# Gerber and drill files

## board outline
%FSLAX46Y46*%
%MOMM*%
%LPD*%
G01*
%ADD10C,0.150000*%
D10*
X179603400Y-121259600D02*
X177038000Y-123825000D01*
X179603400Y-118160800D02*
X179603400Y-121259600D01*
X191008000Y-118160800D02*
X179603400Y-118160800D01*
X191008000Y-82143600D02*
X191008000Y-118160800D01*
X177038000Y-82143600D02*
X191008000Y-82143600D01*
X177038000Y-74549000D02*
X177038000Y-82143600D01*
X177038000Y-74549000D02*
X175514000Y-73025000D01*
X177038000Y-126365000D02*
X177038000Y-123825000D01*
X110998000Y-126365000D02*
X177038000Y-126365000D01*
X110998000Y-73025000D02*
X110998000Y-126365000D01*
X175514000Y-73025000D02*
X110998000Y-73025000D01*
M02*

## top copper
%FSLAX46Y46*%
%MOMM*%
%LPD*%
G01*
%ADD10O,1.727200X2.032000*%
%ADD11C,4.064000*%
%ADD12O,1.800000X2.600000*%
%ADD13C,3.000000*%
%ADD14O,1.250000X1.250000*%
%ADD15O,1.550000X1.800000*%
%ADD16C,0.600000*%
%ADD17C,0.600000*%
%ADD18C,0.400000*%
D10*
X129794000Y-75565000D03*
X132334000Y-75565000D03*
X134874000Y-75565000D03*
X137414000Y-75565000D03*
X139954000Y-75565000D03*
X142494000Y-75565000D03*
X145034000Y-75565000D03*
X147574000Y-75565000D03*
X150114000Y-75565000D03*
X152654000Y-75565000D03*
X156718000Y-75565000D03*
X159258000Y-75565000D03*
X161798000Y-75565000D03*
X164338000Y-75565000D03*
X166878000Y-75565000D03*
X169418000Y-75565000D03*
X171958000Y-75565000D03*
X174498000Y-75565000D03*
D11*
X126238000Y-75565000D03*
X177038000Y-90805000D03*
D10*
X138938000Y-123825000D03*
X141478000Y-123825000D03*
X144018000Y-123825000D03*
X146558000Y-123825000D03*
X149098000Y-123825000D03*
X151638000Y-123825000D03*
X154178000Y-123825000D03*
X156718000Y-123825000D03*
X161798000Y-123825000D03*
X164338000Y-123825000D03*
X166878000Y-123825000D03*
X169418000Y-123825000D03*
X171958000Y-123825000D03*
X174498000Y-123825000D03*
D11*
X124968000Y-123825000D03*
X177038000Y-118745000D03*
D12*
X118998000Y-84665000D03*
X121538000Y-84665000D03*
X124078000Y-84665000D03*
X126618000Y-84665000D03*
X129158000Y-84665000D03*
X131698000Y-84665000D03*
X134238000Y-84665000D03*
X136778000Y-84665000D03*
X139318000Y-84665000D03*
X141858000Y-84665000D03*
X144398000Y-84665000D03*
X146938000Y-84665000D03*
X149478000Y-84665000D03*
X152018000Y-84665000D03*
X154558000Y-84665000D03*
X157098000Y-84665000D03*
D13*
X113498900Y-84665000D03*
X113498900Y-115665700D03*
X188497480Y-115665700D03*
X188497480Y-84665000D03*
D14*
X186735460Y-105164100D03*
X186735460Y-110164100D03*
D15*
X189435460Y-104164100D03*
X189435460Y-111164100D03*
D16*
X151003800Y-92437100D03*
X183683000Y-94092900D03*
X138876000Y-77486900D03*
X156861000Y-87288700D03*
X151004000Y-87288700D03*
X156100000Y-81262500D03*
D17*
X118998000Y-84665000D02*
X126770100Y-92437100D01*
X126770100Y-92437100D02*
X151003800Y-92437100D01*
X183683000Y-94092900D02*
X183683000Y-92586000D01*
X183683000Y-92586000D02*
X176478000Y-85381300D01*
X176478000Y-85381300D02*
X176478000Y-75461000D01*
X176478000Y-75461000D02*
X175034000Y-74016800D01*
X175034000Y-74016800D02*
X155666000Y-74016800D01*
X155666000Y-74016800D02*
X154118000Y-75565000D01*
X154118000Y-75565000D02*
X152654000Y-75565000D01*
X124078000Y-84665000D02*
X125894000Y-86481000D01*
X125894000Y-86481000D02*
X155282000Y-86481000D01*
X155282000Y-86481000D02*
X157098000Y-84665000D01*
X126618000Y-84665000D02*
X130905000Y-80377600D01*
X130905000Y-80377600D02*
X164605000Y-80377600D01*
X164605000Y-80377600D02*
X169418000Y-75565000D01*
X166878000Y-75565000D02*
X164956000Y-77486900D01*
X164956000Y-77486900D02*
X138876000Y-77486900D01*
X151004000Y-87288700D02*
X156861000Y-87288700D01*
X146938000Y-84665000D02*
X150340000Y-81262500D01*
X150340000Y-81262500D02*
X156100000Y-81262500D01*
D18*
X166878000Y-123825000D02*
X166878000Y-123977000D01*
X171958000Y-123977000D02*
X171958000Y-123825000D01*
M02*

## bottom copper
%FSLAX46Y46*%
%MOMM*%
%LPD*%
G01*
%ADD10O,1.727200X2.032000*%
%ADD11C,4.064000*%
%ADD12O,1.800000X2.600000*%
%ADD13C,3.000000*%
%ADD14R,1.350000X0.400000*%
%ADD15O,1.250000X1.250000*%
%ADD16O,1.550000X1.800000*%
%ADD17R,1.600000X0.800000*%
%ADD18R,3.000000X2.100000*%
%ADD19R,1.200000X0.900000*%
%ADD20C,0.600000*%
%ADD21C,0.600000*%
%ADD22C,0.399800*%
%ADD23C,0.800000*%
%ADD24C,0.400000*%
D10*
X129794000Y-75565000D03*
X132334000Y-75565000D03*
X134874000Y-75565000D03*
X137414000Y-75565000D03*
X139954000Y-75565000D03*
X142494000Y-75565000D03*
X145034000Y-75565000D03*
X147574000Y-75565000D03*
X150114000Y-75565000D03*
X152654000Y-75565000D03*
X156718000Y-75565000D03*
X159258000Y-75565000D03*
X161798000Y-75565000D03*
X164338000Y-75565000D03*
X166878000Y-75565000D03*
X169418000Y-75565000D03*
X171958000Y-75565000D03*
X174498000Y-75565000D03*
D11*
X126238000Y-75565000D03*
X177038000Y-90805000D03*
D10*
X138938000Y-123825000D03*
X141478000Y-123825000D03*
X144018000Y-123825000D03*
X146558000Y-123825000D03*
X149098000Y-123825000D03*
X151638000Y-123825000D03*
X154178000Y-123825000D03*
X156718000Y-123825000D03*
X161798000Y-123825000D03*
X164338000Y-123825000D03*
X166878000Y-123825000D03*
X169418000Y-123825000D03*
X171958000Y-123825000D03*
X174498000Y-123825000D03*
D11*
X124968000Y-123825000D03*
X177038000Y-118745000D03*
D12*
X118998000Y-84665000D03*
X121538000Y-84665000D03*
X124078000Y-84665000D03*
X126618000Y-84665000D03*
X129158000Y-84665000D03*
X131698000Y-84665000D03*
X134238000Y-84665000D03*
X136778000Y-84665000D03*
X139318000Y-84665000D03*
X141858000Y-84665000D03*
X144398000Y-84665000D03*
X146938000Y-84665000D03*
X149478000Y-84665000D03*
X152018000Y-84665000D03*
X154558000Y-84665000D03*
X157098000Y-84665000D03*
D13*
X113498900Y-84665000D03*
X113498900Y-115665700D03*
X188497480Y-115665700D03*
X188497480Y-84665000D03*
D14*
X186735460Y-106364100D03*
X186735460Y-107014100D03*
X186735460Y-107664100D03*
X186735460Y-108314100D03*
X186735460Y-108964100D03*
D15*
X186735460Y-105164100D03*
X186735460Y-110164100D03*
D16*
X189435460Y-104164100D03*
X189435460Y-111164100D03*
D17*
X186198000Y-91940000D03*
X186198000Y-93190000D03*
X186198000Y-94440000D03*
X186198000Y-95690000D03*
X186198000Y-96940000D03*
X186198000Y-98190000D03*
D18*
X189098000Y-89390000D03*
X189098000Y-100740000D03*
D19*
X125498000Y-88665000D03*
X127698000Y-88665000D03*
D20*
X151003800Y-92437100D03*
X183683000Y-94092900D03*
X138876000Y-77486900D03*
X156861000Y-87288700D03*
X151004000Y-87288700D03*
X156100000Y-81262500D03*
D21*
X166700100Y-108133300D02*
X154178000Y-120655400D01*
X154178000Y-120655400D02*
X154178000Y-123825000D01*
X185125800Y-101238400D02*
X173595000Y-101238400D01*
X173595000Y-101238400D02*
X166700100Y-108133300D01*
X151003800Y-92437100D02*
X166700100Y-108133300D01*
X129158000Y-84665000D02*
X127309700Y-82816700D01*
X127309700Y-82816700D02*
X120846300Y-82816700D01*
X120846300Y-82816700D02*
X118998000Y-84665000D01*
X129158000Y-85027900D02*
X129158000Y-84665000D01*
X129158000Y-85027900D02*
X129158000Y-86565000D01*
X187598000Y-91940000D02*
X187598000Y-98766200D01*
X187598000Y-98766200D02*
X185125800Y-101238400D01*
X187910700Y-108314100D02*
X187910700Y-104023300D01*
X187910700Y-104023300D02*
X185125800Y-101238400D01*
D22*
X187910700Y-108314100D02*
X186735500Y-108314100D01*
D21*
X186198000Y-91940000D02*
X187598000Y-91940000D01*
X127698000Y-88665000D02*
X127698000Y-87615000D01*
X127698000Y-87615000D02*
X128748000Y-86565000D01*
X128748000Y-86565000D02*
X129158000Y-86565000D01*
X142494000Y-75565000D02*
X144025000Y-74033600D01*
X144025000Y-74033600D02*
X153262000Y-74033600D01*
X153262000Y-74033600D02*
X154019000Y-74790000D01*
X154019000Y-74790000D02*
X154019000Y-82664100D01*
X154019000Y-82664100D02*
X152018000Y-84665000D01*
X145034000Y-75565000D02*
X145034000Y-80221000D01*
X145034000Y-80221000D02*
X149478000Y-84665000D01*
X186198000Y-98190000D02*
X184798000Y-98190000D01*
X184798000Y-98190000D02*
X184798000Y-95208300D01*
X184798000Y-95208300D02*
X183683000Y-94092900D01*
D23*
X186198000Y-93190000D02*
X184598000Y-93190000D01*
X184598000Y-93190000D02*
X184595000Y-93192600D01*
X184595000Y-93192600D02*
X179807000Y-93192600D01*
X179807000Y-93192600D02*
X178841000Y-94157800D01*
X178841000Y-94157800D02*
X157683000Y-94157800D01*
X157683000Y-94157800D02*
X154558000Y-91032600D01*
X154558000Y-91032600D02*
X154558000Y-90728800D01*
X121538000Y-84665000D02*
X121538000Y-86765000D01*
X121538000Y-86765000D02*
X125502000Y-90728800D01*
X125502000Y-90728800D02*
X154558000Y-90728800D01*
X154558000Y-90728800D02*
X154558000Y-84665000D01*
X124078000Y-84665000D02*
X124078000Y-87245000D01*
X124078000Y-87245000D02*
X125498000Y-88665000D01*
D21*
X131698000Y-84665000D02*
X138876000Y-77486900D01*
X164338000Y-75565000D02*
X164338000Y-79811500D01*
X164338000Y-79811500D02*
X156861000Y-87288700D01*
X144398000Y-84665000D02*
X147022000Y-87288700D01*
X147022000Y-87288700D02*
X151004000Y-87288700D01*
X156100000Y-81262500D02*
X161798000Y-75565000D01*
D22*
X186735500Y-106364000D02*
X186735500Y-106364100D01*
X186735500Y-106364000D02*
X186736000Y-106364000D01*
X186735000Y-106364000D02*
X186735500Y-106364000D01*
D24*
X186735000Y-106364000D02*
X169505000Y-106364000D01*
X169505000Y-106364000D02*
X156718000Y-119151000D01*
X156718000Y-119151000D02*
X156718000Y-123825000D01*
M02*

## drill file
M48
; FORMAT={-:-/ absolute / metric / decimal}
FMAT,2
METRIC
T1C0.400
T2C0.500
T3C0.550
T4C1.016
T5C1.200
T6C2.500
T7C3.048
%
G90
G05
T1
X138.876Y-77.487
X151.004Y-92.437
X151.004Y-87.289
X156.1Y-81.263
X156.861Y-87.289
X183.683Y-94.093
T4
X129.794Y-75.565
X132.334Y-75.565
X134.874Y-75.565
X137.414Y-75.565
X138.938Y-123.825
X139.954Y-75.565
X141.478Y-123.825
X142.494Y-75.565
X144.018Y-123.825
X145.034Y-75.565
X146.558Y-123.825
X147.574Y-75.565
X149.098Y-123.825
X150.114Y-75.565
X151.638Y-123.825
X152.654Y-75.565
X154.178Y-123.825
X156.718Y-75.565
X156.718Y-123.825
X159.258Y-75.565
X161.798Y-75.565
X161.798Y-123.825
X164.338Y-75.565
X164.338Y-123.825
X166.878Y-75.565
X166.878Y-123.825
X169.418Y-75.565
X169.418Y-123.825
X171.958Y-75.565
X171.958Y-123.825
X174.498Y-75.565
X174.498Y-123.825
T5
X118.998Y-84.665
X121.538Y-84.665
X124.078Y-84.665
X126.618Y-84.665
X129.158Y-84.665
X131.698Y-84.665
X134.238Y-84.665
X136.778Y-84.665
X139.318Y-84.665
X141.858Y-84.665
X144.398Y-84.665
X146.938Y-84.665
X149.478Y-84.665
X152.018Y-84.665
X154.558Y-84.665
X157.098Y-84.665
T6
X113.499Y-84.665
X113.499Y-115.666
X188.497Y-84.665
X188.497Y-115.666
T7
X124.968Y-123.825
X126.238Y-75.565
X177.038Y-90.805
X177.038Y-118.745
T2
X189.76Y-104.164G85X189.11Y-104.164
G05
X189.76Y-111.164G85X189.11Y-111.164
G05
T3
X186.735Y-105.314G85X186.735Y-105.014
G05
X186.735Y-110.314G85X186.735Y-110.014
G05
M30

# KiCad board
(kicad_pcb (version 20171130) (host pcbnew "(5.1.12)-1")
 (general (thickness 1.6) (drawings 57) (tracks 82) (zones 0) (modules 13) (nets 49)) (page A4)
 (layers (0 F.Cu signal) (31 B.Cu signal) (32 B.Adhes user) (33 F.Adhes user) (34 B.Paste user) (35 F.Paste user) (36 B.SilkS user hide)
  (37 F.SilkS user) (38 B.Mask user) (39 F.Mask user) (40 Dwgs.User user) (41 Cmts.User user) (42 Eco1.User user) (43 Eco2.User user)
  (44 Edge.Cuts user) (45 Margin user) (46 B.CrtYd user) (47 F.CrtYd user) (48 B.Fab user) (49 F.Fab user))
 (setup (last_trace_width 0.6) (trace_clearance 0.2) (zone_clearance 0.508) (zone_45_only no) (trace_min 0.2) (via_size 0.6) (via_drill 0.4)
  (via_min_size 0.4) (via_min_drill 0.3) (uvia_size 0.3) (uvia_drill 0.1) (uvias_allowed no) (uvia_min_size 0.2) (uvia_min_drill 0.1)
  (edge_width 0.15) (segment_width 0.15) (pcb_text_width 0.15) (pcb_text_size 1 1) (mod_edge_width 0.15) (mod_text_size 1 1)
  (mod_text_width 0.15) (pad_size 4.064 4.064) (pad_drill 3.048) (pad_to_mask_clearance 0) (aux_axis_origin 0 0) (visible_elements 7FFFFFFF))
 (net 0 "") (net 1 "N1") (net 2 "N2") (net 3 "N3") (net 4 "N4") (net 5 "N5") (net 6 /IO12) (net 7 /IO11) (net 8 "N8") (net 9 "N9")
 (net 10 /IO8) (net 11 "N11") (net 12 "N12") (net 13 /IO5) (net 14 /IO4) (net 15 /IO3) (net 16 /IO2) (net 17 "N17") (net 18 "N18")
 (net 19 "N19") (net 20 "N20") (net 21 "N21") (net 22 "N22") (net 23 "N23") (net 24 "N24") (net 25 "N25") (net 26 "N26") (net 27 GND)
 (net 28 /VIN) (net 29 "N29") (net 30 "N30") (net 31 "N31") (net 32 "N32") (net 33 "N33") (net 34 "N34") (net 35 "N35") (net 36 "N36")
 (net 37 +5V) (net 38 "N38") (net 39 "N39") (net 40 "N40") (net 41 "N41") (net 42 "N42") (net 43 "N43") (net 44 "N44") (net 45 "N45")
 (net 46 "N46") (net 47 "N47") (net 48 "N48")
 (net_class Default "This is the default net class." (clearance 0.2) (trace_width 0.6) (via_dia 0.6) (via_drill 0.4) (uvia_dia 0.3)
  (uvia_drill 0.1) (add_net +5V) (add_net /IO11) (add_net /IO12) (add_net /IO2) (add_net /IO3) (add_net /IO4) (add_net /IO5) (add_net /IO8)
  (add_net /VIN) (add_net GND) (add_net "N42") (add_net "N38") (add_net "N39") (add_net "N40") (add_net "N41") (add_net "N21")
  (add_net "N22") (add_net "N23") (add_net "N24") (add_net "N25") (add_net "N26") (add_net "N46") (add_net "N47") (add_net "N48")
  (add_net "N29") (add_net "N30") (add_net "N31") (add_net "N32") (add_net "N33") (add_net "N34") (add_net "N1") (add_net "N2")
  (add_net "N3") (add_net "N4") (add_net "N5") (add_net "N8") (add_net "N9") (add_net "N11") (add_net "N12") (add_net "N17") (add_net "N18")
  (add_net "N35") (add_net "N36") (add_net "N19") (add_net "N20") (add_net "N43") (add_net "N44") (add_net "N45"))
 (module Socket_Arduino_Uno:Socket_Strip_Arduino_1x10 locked (layer F.Cu) (at 129.794 75.565)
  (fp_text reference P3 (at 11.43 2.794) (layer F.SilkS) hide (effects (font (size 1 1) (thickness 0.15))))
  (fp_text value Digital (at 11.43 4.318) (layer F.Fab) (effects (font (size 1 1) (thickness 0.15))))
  (pad 1 thru_hole oval (at 0 0) (size 1.7272 2.032) (drill 1.016) (layers *.Cu *.Mask F.SilkS) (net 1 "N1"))
  (pad 2 thru_hole oval (at 2.54 0) (size 1.7272 2.032) (drill 1.016) (layers *.Cu *.Mask F.SilkS) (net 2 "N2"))
  (pad 3 thru_hole oval (at 5.08 0) (size 1.7272 2.032) (drill 1.016) (layers *.Cu *.Mask F.SilkS) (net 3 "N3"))
  (pad 4 thru_hole oval (at 7.62 0) (size 1.7272 2.032) (drill 1.016) (layers *.Cu *.Mask F.SilkS) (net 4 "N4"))
  (pad 5 thru_hole oval (at 10.16 0) (size 1.7272 2.032) (drill 1.016) (layers *.Cu *.Mask F.SilkS) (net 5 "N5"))
  (pad 6 thru_hole oval (at 12.7 0) (size 1.7272 2.032) (drill 1.016) (layers *.Cu *.Mask F.SilkS) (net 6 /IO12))
  (pad 7 thru_hole oval (at 15.24 0) (size 1.7272 2.032) (drill 1.016) (layers *.Cu *.Mask F.SilkS) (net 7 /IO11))
  (pad 8 thru_hole oval (at 17.78 0) (size 1.7272 2.032) (drill 1.016) (layers *.Cu *.Mask F.SilkS) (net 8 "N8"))
  (pad 9 thru_hole oval (at 20.32 0) (size 1.7272 2.032) (drill 1.016) (layers *.Cu *.Mask F.SilkS) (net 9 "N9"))
  (pad 10 thru_hole oval (at 22.86 0) (size 1.7272 2.032) (drill 1.016) (layers *.Cu *.Mask F.SilkS) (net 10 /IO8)))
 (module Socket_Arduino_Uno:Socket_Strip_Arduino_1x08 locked (layer F.Cu) (at 156.718 75.565)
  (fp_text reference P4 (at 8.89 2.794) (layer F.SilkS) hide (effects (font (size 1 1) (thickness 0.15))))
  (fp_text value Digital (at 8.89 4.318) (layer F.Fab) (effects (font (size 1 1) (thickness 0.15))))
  (pad 1 thru_hole oval (at 0 0) (size 1.7272 2.032) (drill 1.016) (layers *.Cu *.Mask F.SilkS) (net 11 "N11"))
  (pad 2 thru_hole oval (at 2.54 0) (size 1.7272 2.032) (drill 1.016) (layers *.Cu *.Mask F.SilkS) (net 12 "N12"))
  (pad 3 thru_hole oval (at 5.08 0) (size 1.7272 2.032) (drill 1.016) (layers *.Cu *.Mask F.SilkS) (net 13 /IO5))
  (pad 4 thru_hole oval (at 7.62 0) (size 1.7272 2.032) (drill 1.016) (layers *.Cu *.Mask F.SilkS) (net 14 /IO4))
  (pad 5 thru_hole oval (at 10.16 0) (size 1.7272 2.032) (drill 1.016) (layers *.Cu *.Mask F.SilkS) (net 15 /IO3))
  (pad 6 thru_hole oval (at 12.7 0) (size 1.7272 2.032) (drill 1.016) (layers *.Cu *.Mask F.SilkS) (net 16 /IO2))
  (pad 7 thru_hole oval (at 15.24 0) (size 1.7272 2.032) (drill 1.016) (layers *.Cu *.Mask F.SilkS) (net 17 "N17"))
  (pad 8 thru_hole oval (at 17.78 0) (size 1.7272 2.032) (drill 1.016) (layers *.Cu *.Mask F.SilkS) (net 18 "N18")))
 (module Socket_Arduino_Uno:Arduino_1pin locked (layer F.Cu) (at 126.238 75.565)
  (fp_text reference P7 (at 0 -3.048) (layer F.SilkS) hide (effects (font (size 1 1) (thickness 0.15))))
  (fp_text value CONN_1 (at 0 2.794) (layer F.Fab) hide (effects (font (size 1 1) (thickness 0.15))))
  (pad 1 thru_hole circle (at 0 0) (size 4.064 4.064) (drill 3.048) (layers *.Cu *.Mask F.SilkS) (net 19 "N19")))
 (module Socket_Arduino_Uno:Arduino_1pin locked (layer F.Cu) (at 177.038 90.805)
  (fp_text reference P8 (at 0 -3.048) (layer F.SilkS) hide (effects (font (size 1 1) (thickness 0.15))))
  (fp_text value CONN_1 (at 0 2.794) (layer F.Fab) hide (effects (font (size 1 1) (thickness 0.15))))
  (pad 1 thru_hole circle (at 0 0) (size 4.064 4.064) (drill 3.048) (layers *.Cu *.Mask F.SilkS) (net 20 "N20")))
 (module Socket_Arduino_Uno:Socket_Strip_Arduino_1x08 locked (layer F.Cu) (at 138.938 123.825)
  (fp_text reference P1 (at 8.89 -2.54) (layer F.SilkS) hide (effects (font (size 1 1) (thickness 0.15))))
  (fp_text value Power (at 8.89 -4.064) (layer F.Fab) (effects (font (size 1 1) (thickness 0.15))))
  (pad 1 thru_hole oval (at 0 0) (size 1.7272 2.032) (drill 1.016) (layers *.Cu *.Mask F.SilkS) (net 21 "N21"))
  (pad 2 thru_hole oval (at 2.54 0) (size 1.7272 2.032) (drill 1.016) (layers *.Cu *.Mask F.SilkS) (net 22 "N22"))
  (pad 3 thru_hole oval (at 5.08 0) (size 1.7272 2.032) (drill 1.016) (layers *.Cu *.Mask F.SilkS) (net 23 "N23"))
  (pad 4 thru_hole oval (at 7.62 0) (size 1.7272 2.032) (drill 1.016) (layers *.Cu *.Mask F.SilkS) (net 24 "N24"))
  (pad 5 thru_hole oval (at 10.16 0) (size 1.7272 2.032) (drill 1.016) (layers *.Cu *.Mask F.SilkS) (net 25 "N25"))
  (pad 6 thru_hole oval (at 12.7 0) (size 1.7272 2.032) (drill 1.016) (layers *.Cu *.Mask F.SilkS) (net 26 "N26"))
  (pad 7 thru_hole oval (at 15.24 0) (size 1.7272 2.032) (drill 1.016) (layers *.Cu *.Mask F.SilkS) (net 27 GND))
  (pad 8 thru_hole oval (at 17.78 0) (size 1.7272 2.032) (drill 1.016) (layers *.Cu *.Mask F.SilkS) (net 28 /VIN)))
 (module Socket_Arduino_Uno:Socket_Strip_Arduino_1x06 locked (layer F.Cu) (at 161.798 123.825)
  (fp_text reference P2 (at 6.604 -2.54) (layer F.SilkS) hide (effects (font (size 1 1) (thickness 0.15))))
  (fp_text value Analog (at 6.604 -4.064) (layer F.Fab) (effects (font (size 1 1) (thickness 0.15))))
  (pad 1 thru_hole oval (at 0 0) (size 1.7272 2.032) (drill 1.016) (layers *.Cu *.Mask F.SilkS) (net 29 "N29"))
  (pad 2 thru_hole oval (at 2.54 0) (size 1.7272 2.032) (drill 1.016) (layers *.Cu *.Mask F.SilkS) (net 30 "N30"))
  (pad 3 thru_hole oval (at 5.08 0) (size 1.7272 2.032) (drill 1.016) (layers *.Cu *.Mask F.SilkS) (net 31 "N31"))
  (pad 4 thru_hole oval (at 7.62 0) (size 1.7272 2.032) (drill 1.016) (layers *.Cu *.Mask F.SilkS) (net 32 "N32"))
  (pad 5 thru_hole oval (at 10.16 0) (size 1.7272 2.032) (drill 1.016) (layers *.Cu *.Mask F.SilkS) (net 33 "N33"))
  (pad 6 thru_hole oval (at 12.7 0) (size 1.7272 2.032) (drill 1.016) (layers *.Cu *.Mask F.SilkS) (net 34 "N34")))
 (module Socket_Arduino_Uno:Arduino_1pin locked (layer F.Cu) (at 124.968 123.825)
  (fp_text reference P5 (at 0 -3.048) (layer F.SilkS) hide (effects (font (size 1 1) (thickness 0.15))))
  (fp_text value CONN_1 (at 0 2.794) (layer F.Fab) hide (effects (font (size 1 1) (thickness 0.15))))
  (pad 1 thru_hole circle (at 0 0) (size 4.064 4.064) (drill 3.048) (layers *.Cu *.Mask F.SilkS) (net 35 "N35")))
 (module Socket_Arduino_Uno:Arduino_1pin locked (layer F.Cu) (at 177.038 118.745)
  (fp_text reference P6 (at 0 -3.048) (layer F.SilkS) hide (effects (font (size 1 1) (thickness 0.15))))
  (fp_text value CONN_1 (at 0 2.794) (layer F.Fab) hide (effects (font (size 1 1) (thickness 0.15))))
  (pad 1 thru_hole circle (at 0 0) (size 4.064 4.064) (drill 3.048) (layers *.Cu *.Mask F.SilkS) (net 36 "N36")))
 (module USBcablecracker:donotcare (layer B.Cu) (at 164.1856 107.3658 180)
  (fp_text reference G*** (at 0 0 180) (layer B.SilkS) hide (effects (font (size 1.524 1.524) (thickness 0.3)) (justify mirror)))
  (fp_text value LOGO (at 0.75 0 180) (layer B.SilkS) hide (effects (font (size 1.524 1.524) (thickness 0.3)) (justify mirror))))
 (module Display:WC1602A (layer F.Cu) (at 118.998 84.665)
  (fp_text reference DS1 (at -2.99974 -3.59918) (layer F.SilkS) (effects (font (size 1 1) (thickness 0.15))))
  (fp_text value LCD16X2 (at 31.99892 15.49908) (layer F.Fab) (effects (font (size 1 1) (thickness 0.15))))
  (pad 1 thru_hole oval (at 0 0) (size 1.8 2.6) (drill 1.2) (layers *.Cu *.Mask F.SilkS) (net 27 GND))
  (pad 2 thru_hole oval (at 2.54 0) (size 1.8 2.6) (drill 1.2) (layers *.Cu *.Mask F.SilkS) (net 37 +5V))
  (pad 3 thru_hole oval (at 5.08 0) (size 1.8 2.6) (drill 1.2) (layers *.Cu *.Mask F.SilkS) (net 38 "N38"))
  (pad 4 thru_hole oval (at 7.62 0) (size 1.8 2.6) (drill 1.2) (layers *.Cu *.Mask F.SilkS) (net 16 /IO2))
  (pad 5 thru_hole oval (at 10.16 0) (size 1.8 2.6) (drill 1.2) (layers *.Cu *.Mask F.SilkS) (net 27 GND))
  (pad 6 thru_hole oval (at 12.7 0) (size 1.8 2.6) (drill 1.2) (layers *.Cu *.Mask F.SilkS) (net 15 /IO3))
  (pad 7 thru_hole oval (at 15.24 0) (size 1.8 2.6) (drill 1.2) (layers *.Cu *.Mask F.SilkS) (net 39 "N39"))
  (pad 8 thru_hole oval (at 17.78 0) (size 1.8 2.6) (drill 1.2) (layers *.Cu *.Mask F.SilkS) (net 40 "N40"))
  (pad 9 thru_hole oval (at 20.32 0) (size 1.8 2.6) (drill 1.2) (layers *.Cu *.Mask F.SilkS) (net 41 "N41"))
  (pad 10 thru_hole oval (at 22.86 0) (size 1.8 2.6) (drill 1.2) (layers *.Cu *.Mask F.SilkS) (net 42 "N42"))
  (pad 11 thru_hole oval (at 25.4 0) (size 1.8 2.6) (drill 1.2) (layers *.Cu *.Mask F.SilkS) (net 14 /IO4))
  (pad 12 thru_hole oval (at 27.94 0) (size 1.8 2.6) (drill 1.2) (layers *.Cu *.Mask F.SilkS) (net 13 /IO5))
  (pad 13 thru_hole oval (at 30.48 0) (size 1.8 2.6) (drill 1.2) (layers *.Cu *.Mask F.SilkS) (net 7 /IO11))
  (pad 14 thru_hole oval (at 33.02 0) (size 1.8 2.6) (drill 1.2) (layers *.Cu *.Mask F.SilkS) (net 6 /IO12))
  (pad 15 thru_hole oval (at 35.56 0) (size 1.8 2.6) (drill 1.2) (layers *.Cu *.Mask F.SilkS) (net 37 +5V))
  (pad 16 thru_hole oval (at 38.1 0) (size 1.8 2.6) (drill 1.2) (layers *.Cu *.Mask F.SilkS) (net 38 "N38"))
  (pad 0 thru_hole circle (at -5.4991 0) (size 3 3) (drill 2.5) (layers *.Cu *.Mask F.SilkS))
  (pad 0 thru_hole circle (at -5.4991 31.0007) (size 3 3) (drill 2.5) (layers *.Cu *.Mask F.SilkS))
  (pad 0 thru_hole circle (at 69.49948 31.0007) (size 3 3) (drill 2.5) (layers *.Cu *.Mask F.SilkS))
  (pad 0 thru_hole circle (at 69.49948 0) (size 3 3) (drill 2.5) (layers *.Cu *.Mask F.SilkS)))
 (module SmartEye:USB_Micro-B (layer B.Cu) (at 188.298 107.665 270)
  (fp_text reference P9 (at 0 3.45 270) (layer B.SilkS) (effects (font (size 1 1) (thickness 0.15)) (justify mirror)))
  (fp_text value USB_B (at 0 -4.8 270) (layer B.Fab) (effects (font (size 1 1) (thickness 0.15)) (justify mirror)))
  (pad 1 smd rect (at -1.3009 1.56254 180) (size 1.35 0.4) (layers B.Cu B.Paste B.Mask) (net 28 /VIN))
  (pad 2 smd rect (at -0.6509 1.56254 180) (size 1.35 0.4) (layers B.Cu B.Paste B.Mask) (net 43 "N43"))
  (pad 3 smd rect (at -0.0009 1.56254 180) (size 1.35 0.4) (layers B.Cu B.Paste B.Mask) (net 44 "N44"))
  (pad 4 smd rect (at 0.6491 1.56254 180) (size 1.35 0.4) (layers B.Cu B.Paste B.Mask) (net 27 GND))
  (pad 5 smd rect (at 1.2991 1.56254 180) (size 1.35 0.4) (layers B.Cu B.Paste B.Mask) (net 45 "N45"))
  (pad 6 thru_hole oval (at -2.5009 1.56254 180) (size 1.25 1.25) (drill oval 0.55 0.85) (layers *.Cu *.Mask B.SilkS))
  (pad 6 thru_hole oval (at 2.4991 1.56254 180) (size 1.25 1.25) (drill oval 0.55 0.85) (layers *.Cu *.Mask B.SilkS))
  (pad 6 thru_hole oval (at -3.5009 -1.13746 180) (size 1.55 1.8) (drill oval 1.15 0.5) (layers *.Cu *.Mask B.SilkS))
  (pad 6 thru_hole oval (at 3.4991 -1.13746 180) (size 1.55 1.8) (drill oval 1.15 0.5) (layers *.Cu *.Mask B.SilkS)))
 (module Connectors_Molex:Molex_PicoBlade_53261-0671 (layer B.Cu) (at 189.098 95.065 270)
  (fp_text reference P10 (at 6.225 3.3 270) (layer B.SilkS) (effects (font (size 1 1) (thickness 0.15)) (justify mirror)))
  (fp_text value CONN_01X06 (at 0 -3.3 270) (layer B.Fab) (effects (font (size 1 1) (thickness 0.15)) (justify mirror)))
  (pad 1 smd rect (at -3.125 2.9 270) (size 0.8 1.6) (layers B.Cu B.Paste B.Mask) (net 27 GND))
  (pad 2 smd rect (at -1.875 2.9 270) (size 0.8 1.6) (layers B.Cu B.Paste B.Mask) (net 37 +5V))
  (pad 3 smd rect (at -0.625 2.9 270) (size 0.8 1.6) (layers B.Cu B.Paste B.Mask) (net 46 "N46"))
  (pad 4 smd rect (at 0.625 2.9 270) (size 0.8 1.6) (layers B.Cu B.Paste B.Mask) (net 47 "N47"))
  (pad 5 smd rect (at 1.875 2.9 270) (size 0.8 1.6) (layers B.Cu B.Paste B.Mask) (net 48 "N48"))
  (pad 6 smd rect (at 3.125 2.9 270) (size 0.8 1.6) (layers B.Cu B.Paste B.Mask) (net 10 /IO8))
  (pad "" smd rect (at -5.675 0 270) (size 2.1 3) (layers B.Cu B.Paste B.Mask))
  (pad "" smd rect (at 5.675 0 270) (size 2.1 3) (layers B.Cu B.Paste B.Mask)))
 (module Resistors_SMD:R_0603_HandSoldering (layer B.Cu) (at 126.598 88.665)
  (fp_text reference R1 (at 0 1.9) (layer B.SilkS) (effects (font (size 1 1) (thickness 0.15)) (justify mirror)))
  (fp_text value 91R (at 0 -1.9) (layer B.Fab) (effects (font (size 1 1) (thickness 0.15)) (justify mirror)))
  (pad 1 smd rect (at -1.1 0) (size 1.2 0.9) (layers B.Cu B.Paste B.Mask) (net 38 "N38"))
  (pad 2 smd rect (at 1.1 0) (size 1.2 0.9) (layers B.Cu B.Paste B.Mask) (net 27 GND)))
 (gr_line (start 179.6034 121.2596) (end 177.038 123.825) (angle 90) (layer Edge.Cuts) (width 0.15))
 (gr_line (start 179.6034 118.1608) (end 179.6034 121.2596) (angle 90) (layer Edge.Cuts) (width 0.15))
 (gr_line (start 191.008 118.1608) (end 179.6034 118.1608) (angle 90) (layer Edge.Cuts) (width 0.15))
 (gr_line (start 191.008 82.1436) (end 191.008 118.1608) (angle 90) (layer Edge.Cuts) (width 0.15))
 (gr_line (start 177.038 82.1436) (end 191.008 82.1436) (angle 90) (layer Edge.Cuts) (width 0.15))
 (gr_line (start 177.038 74.549) (end 177.038 82.1436) (angle 90) (layer Edge.Cuts) (width 0.15))
 (gr_line (start 177.038 74.549) (end 175.514 73.025) (angle 90) (layer Edge.Cuts) (width 0.15))
 (gr_line (start 177.038 126.365) (end 177.038 123.825) (angle 90) (layer Edge.Cuts) (width 0.15))
 (gr_line (start 110.998 126.365) (end 177.038 126.365) (angle 90) (layer Edge.Cuts) (width 0.15))
 (gr_line (start 110.998 73.025) (end 110.998 126.365) (angle 90) (layer Edge.Cuts) (width 0.15))
 (gr_line (start 175.514 73.025) (end 110.998 73.025) (angle 90) (layer Edge.Cuts) (width 0.15))
 (segment (start 166.7001 108.1333) (end 154.178 120.6554) (width 0.6) (layer B.Cu) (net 27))
 (segment (start 154.178 120.6554) (end 154.178 123.825) (width 0.6) (layer B.Cu) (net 27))
 (segment (start 185.1258 101.2384) (end 173.595 101.2384) (width 0.6) (layer B.Cu) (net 27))
 (segment (start 173.595 101.2384) (end 166.7001 108.1333) (width 0.6) (layer B.Cu) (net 27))
 (segment (start 151.0038 92.4371) (end 166.7001 108.1333) (width 0.6) (layer B.Cu) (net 27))
 (segment (start 118.998 84.665) (end 126.7701 92.4371) (width 0.6) (layer F.Cu) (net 27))
 (segment (start 126.7701 92.4371) (end 151.0038 92.4371) (width 0.6) (layer F.Cu) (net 27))
 (segment (start 129.158 84.665) (end 127.3097 82.8167) (width 0.6) (layer B.Cu) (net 27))
 (segment (start 127.3097 82.8167) (end 120.8463 82.8167) (width 0.6) (layer B.Cu) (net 27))
 (segment (start 120.8463 82.8167) (end 118.998 84.665) (width 0.6) (layer B.Cu) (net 27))
 (segment (start 129.158 85.0279) (end 129.158 84.665) (width 0.6) (layer B.Cu) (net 27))
 (segment (start 129.158 85.0279) (end 129.158 86.565) (width 0.6) (layer B.Cu) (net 27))
 (segment (start 187.598 91.94) (end 187.598 98.7662) (width 0.6) (layer B.Cu) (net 27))
 (segment (start 187.598 98.7662) (end 185.1258 101.2384) (width 0.6) (layer B.Cu) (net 27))
 (segment (start 187.9107 108.3141) (end 187.9107 104.0233) (width 0.6) (layer B.Cu) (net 27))
 (segment (start 187.9107 104.0233) (end 185.1258 101.2384) (width 0.6) (layer B.Cu) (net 27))
 (segment (start 187.9107 108.3141) (end 186.7355 108.3141) (width 0.3998) (layer B.Cu) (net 27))
 (segment (start 186.198 91.94) (end 187.598 91.94) (width 0.6) (layer B.Cu) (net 27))
 (segment (start 127.698 88.665) (end 127.698 87.615) (width 0.6) (layer B.Cu) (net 27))
 (segment (start 127.698 87.615) (end 128.748 86.565) (width 0.6) (layer B.Cu) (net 27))
 (segment (start 128.748 86.565) (end 129.158 86.565) (width 0.6) (layer B.Cu) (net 27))
 (via (at 151.0038 92.4371) (size 0.6) (layers F.Cu B.Cu) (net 27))
 (segment (start 142.494 75.565) (end 144.025 74.0336) (width 0.6) (layer B.Cu) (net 6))
 (segment (start 144.025 74.0336) (end 153.262 74.0336) (width 0.6) (layer B.Cu) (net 6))
 (segment (start 153.262 74.0336) (end 154.019 74.79) (width 0.6) (layer B.Cu) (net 6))
 (segment (start 154.019 74.79) (end 154.019 82.6641) (width 0.6) (layer B.Cu) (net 6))
 (segment (start 154.019 82.6641) (end 152.018 84.665) (width 0.6) (layer B.Cu) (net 6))
 (segment (start 145.034 75.565) (end 145.034 80.221) (width 0.6) (layer B.Cu) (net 7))
 (segment (start 145.034 80.221) (end 149.478 84.665) (width 0.6) (layer B.Cu) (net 7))
 (segment (start 186.198 98.19) (end 184.798 98.19) (width 0.6) (layer B.Cu) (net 10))
 (segment (start 184.798 98.19) (end 184.798 95.2083) (width 0.6) (layer B.Cu) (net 10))
 (segment (start 184.798 95.2083) (end 183.683 94.0929) (width 0.6) (layer B.Cu) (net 10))
 (segment (start 183.683 94.0929) (end 183.683 92.586) (width 0.6) (layer F.Cu) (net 10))
 (segment (start 183.683 92.586) (end 176.478 85.3813) (width 0.6) (layer F.Cu) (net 10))
 (segment (start 176.478 85.3813) (end 176.478 75.461) (width 0.6) (layer F.Cu) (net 10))
 (segment (start 176.478 75.461) (end 175.034 74.0168) (width 0.6) (layer F.Cu) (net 10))
 (segment (start 175.034 74.0168) (end 155.666 74.0168) (width 0.6) (layer F.Cu) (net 10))
 (segment (start 155.666 74.0168) (end 154.118 75.565) (width 0.6) (layer F.Cu) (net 10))
 (segment (start 154.118 75.565) (end 152.654 75.565) (width 0.6) (layer F.Cu) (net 10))
 (via (at 183.683 94.0929) (size 0.6) (layers F.Cu B.Cu) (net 10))
 (segment (start 186.198 93.19) (end 184.598 93.19) (width 0.8) (layer B.Cu) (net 37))
 (segment (start 184.598 93.19) (end 184.595 93.1926) (width 0.8) (layer B.Cu) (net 37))
 (segment (start 184.595 93.1926) (end 179.807 93.1926) (width 0.8) (layer B.Cu) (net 37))
 (segment (start 179.807 93.1926) (end 178.841 94.1578) (width 0.8) (layer B.Cu) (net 37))
 (segment (start 178.841 94.1578) (end 157.683 94.1578) (width 0.8) (layer B.Cu) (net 37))
 (segment (start 157.683 94.1578) (end 154.558 91.0326) (width 0.8) (layer B.Cu) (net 37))
 (segment (start 154.558 91.0326) (end 154.558 90.7288) (width 0.8) (layer B.Cu) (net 37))
 (segment (start 121.538 84.665) (end 121.538 86.765) (width 0.8) (layer B.Cu) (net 37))
 (segment (start 121.538 86.765) (end 125.502 90.7288) (width 0.8) (layer B.Cu) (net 37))
 (segment (start 125.502 90.7288) (end 154.558 90.7288) (width 0.8) (layer B.Cu) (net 37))
 (segment (start 154.558 90.7288) (end 154.558 84.665) (width 0.8) (layer B.Cu) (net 37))
 (segment (start 124.078 84.665) (end 125.894 86.481) (width 0.6) (layer F.Cu) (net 38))
 (segment (start 125.894 86.481) (end 155.282 86.481) (width 0.6) (layer F.Cu) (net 38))
 (segment (start 155.282 86.481) (end 157.098 84.665) (width 0.6) (layer F.Cu) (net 38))
 (segment (start 124.078 84.665) (end 124.078 87.245) (width 0.8) (layer B.Cu) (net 38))
 (segment (start 124.078 87.245) (end 125.498 88.665) (width 0.8) (layer B.Cu) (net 38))
 (segment (start 126.618 84.665) (end 130.905 80.3776) (width 0.6) (layer F.Cu) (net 16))
 (segment (start 130.905 80.3776) (end 164.605 80.3776) (width 0.6) (layer F.Cu) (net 16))
 (segment (start 164.605 80.3776) (end 169.418 75.565) (width 0.6) (layer F.Cu) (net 16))
 (segment (start 166.878 75.565) (end 164.956 77.4869) (width 0.6) (layer F.Cu) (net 15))
 (segment (start 164.956 77.4869) (end 138.876 77.4869) (width 0.6) (layer F.Cu) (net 15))
 (segment (start 131.698 84.665) (end 138.876 77.4869) (width 0.6) (layer B.Cu) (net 15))
 (via (at 138.876 77.4869) (size 0.6) (layers F.Cu B.Cu) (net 15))
 (segment (start 151.004 87.2887) (end 156.861 87.2887) (width 0.6) (layer F.Cu) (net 14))
 (segment (start 164.338 75.565) (end 164.338 79.8115) (width 0.6) (layer B.Cu) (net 14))
 (segment (start 164.338 79.8115) (end 156.861 87.2887) (width 0.6) (layer B.Cu) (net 14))
 (segment (start 144.398 84.665) (end 147.022 87.2887) (width 0.6) (layer B.Cu) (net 14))
 (segment (start 147.022 87.2887) (end 151.004 87.2887) (width 0.6) (layer B.Cu) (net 14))
 (via (at 156.861 87.2887) (size 0.6) (layers F.Cu B.Cu) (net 14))
 (via (at 151.004 87.2887) (size 0.6) (layers F.Cu B.Cu) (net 14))
 (segment (start 146.938 84.665) (end 150.34 81.2625) (width 0.6) (layer F.Cu) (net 13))
 (segment (start 150.34 81.2625) (end 156.1 81.2625) (width 0.6) (layer F.Cu) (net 13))
 (segment (start 156.1 81.2625) (end 161.798 75.565) (width 0.6) (layer B.Cu) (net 13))
 (via (at 156.1 81.2625) (size 0.6) (layers F.Cu B.Cu) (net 13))
 (segment (start 186.7355 106.364) (end 186.7355 106.3641) (width 0.3998) (layer B.Cu) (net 28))
 (segment (start 186.7355 106.364) (end 186.736 106.364) (width 0.3998) (layer B.Cu) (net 28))
 (segment (start 186.735 106.364) (end 186.7355 106.364) (width 0.3998) (layer B.Cu) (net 28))
 (segment (start 186.735 106.364) (end 169.505 106.364) (width 0.4) (layer B.Cu) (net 28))
 (segment (start 169.505 106.364) (end 156.718 119.151) (width 0.4) (layer B.Cu) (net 28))
 (segment (start 156.718 119.151) (end 156.718 123.825) (width 0.4) (layer B.Cu) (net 28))
 (segment (start 166.878 123.825) (end 166.878 123.977) (width 0.4) (layer F.Cu) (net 31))
 (segment (start 171.958 123.977) (end 171.958 123.825) (width 0.4) (layer F.Cu) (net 33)))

